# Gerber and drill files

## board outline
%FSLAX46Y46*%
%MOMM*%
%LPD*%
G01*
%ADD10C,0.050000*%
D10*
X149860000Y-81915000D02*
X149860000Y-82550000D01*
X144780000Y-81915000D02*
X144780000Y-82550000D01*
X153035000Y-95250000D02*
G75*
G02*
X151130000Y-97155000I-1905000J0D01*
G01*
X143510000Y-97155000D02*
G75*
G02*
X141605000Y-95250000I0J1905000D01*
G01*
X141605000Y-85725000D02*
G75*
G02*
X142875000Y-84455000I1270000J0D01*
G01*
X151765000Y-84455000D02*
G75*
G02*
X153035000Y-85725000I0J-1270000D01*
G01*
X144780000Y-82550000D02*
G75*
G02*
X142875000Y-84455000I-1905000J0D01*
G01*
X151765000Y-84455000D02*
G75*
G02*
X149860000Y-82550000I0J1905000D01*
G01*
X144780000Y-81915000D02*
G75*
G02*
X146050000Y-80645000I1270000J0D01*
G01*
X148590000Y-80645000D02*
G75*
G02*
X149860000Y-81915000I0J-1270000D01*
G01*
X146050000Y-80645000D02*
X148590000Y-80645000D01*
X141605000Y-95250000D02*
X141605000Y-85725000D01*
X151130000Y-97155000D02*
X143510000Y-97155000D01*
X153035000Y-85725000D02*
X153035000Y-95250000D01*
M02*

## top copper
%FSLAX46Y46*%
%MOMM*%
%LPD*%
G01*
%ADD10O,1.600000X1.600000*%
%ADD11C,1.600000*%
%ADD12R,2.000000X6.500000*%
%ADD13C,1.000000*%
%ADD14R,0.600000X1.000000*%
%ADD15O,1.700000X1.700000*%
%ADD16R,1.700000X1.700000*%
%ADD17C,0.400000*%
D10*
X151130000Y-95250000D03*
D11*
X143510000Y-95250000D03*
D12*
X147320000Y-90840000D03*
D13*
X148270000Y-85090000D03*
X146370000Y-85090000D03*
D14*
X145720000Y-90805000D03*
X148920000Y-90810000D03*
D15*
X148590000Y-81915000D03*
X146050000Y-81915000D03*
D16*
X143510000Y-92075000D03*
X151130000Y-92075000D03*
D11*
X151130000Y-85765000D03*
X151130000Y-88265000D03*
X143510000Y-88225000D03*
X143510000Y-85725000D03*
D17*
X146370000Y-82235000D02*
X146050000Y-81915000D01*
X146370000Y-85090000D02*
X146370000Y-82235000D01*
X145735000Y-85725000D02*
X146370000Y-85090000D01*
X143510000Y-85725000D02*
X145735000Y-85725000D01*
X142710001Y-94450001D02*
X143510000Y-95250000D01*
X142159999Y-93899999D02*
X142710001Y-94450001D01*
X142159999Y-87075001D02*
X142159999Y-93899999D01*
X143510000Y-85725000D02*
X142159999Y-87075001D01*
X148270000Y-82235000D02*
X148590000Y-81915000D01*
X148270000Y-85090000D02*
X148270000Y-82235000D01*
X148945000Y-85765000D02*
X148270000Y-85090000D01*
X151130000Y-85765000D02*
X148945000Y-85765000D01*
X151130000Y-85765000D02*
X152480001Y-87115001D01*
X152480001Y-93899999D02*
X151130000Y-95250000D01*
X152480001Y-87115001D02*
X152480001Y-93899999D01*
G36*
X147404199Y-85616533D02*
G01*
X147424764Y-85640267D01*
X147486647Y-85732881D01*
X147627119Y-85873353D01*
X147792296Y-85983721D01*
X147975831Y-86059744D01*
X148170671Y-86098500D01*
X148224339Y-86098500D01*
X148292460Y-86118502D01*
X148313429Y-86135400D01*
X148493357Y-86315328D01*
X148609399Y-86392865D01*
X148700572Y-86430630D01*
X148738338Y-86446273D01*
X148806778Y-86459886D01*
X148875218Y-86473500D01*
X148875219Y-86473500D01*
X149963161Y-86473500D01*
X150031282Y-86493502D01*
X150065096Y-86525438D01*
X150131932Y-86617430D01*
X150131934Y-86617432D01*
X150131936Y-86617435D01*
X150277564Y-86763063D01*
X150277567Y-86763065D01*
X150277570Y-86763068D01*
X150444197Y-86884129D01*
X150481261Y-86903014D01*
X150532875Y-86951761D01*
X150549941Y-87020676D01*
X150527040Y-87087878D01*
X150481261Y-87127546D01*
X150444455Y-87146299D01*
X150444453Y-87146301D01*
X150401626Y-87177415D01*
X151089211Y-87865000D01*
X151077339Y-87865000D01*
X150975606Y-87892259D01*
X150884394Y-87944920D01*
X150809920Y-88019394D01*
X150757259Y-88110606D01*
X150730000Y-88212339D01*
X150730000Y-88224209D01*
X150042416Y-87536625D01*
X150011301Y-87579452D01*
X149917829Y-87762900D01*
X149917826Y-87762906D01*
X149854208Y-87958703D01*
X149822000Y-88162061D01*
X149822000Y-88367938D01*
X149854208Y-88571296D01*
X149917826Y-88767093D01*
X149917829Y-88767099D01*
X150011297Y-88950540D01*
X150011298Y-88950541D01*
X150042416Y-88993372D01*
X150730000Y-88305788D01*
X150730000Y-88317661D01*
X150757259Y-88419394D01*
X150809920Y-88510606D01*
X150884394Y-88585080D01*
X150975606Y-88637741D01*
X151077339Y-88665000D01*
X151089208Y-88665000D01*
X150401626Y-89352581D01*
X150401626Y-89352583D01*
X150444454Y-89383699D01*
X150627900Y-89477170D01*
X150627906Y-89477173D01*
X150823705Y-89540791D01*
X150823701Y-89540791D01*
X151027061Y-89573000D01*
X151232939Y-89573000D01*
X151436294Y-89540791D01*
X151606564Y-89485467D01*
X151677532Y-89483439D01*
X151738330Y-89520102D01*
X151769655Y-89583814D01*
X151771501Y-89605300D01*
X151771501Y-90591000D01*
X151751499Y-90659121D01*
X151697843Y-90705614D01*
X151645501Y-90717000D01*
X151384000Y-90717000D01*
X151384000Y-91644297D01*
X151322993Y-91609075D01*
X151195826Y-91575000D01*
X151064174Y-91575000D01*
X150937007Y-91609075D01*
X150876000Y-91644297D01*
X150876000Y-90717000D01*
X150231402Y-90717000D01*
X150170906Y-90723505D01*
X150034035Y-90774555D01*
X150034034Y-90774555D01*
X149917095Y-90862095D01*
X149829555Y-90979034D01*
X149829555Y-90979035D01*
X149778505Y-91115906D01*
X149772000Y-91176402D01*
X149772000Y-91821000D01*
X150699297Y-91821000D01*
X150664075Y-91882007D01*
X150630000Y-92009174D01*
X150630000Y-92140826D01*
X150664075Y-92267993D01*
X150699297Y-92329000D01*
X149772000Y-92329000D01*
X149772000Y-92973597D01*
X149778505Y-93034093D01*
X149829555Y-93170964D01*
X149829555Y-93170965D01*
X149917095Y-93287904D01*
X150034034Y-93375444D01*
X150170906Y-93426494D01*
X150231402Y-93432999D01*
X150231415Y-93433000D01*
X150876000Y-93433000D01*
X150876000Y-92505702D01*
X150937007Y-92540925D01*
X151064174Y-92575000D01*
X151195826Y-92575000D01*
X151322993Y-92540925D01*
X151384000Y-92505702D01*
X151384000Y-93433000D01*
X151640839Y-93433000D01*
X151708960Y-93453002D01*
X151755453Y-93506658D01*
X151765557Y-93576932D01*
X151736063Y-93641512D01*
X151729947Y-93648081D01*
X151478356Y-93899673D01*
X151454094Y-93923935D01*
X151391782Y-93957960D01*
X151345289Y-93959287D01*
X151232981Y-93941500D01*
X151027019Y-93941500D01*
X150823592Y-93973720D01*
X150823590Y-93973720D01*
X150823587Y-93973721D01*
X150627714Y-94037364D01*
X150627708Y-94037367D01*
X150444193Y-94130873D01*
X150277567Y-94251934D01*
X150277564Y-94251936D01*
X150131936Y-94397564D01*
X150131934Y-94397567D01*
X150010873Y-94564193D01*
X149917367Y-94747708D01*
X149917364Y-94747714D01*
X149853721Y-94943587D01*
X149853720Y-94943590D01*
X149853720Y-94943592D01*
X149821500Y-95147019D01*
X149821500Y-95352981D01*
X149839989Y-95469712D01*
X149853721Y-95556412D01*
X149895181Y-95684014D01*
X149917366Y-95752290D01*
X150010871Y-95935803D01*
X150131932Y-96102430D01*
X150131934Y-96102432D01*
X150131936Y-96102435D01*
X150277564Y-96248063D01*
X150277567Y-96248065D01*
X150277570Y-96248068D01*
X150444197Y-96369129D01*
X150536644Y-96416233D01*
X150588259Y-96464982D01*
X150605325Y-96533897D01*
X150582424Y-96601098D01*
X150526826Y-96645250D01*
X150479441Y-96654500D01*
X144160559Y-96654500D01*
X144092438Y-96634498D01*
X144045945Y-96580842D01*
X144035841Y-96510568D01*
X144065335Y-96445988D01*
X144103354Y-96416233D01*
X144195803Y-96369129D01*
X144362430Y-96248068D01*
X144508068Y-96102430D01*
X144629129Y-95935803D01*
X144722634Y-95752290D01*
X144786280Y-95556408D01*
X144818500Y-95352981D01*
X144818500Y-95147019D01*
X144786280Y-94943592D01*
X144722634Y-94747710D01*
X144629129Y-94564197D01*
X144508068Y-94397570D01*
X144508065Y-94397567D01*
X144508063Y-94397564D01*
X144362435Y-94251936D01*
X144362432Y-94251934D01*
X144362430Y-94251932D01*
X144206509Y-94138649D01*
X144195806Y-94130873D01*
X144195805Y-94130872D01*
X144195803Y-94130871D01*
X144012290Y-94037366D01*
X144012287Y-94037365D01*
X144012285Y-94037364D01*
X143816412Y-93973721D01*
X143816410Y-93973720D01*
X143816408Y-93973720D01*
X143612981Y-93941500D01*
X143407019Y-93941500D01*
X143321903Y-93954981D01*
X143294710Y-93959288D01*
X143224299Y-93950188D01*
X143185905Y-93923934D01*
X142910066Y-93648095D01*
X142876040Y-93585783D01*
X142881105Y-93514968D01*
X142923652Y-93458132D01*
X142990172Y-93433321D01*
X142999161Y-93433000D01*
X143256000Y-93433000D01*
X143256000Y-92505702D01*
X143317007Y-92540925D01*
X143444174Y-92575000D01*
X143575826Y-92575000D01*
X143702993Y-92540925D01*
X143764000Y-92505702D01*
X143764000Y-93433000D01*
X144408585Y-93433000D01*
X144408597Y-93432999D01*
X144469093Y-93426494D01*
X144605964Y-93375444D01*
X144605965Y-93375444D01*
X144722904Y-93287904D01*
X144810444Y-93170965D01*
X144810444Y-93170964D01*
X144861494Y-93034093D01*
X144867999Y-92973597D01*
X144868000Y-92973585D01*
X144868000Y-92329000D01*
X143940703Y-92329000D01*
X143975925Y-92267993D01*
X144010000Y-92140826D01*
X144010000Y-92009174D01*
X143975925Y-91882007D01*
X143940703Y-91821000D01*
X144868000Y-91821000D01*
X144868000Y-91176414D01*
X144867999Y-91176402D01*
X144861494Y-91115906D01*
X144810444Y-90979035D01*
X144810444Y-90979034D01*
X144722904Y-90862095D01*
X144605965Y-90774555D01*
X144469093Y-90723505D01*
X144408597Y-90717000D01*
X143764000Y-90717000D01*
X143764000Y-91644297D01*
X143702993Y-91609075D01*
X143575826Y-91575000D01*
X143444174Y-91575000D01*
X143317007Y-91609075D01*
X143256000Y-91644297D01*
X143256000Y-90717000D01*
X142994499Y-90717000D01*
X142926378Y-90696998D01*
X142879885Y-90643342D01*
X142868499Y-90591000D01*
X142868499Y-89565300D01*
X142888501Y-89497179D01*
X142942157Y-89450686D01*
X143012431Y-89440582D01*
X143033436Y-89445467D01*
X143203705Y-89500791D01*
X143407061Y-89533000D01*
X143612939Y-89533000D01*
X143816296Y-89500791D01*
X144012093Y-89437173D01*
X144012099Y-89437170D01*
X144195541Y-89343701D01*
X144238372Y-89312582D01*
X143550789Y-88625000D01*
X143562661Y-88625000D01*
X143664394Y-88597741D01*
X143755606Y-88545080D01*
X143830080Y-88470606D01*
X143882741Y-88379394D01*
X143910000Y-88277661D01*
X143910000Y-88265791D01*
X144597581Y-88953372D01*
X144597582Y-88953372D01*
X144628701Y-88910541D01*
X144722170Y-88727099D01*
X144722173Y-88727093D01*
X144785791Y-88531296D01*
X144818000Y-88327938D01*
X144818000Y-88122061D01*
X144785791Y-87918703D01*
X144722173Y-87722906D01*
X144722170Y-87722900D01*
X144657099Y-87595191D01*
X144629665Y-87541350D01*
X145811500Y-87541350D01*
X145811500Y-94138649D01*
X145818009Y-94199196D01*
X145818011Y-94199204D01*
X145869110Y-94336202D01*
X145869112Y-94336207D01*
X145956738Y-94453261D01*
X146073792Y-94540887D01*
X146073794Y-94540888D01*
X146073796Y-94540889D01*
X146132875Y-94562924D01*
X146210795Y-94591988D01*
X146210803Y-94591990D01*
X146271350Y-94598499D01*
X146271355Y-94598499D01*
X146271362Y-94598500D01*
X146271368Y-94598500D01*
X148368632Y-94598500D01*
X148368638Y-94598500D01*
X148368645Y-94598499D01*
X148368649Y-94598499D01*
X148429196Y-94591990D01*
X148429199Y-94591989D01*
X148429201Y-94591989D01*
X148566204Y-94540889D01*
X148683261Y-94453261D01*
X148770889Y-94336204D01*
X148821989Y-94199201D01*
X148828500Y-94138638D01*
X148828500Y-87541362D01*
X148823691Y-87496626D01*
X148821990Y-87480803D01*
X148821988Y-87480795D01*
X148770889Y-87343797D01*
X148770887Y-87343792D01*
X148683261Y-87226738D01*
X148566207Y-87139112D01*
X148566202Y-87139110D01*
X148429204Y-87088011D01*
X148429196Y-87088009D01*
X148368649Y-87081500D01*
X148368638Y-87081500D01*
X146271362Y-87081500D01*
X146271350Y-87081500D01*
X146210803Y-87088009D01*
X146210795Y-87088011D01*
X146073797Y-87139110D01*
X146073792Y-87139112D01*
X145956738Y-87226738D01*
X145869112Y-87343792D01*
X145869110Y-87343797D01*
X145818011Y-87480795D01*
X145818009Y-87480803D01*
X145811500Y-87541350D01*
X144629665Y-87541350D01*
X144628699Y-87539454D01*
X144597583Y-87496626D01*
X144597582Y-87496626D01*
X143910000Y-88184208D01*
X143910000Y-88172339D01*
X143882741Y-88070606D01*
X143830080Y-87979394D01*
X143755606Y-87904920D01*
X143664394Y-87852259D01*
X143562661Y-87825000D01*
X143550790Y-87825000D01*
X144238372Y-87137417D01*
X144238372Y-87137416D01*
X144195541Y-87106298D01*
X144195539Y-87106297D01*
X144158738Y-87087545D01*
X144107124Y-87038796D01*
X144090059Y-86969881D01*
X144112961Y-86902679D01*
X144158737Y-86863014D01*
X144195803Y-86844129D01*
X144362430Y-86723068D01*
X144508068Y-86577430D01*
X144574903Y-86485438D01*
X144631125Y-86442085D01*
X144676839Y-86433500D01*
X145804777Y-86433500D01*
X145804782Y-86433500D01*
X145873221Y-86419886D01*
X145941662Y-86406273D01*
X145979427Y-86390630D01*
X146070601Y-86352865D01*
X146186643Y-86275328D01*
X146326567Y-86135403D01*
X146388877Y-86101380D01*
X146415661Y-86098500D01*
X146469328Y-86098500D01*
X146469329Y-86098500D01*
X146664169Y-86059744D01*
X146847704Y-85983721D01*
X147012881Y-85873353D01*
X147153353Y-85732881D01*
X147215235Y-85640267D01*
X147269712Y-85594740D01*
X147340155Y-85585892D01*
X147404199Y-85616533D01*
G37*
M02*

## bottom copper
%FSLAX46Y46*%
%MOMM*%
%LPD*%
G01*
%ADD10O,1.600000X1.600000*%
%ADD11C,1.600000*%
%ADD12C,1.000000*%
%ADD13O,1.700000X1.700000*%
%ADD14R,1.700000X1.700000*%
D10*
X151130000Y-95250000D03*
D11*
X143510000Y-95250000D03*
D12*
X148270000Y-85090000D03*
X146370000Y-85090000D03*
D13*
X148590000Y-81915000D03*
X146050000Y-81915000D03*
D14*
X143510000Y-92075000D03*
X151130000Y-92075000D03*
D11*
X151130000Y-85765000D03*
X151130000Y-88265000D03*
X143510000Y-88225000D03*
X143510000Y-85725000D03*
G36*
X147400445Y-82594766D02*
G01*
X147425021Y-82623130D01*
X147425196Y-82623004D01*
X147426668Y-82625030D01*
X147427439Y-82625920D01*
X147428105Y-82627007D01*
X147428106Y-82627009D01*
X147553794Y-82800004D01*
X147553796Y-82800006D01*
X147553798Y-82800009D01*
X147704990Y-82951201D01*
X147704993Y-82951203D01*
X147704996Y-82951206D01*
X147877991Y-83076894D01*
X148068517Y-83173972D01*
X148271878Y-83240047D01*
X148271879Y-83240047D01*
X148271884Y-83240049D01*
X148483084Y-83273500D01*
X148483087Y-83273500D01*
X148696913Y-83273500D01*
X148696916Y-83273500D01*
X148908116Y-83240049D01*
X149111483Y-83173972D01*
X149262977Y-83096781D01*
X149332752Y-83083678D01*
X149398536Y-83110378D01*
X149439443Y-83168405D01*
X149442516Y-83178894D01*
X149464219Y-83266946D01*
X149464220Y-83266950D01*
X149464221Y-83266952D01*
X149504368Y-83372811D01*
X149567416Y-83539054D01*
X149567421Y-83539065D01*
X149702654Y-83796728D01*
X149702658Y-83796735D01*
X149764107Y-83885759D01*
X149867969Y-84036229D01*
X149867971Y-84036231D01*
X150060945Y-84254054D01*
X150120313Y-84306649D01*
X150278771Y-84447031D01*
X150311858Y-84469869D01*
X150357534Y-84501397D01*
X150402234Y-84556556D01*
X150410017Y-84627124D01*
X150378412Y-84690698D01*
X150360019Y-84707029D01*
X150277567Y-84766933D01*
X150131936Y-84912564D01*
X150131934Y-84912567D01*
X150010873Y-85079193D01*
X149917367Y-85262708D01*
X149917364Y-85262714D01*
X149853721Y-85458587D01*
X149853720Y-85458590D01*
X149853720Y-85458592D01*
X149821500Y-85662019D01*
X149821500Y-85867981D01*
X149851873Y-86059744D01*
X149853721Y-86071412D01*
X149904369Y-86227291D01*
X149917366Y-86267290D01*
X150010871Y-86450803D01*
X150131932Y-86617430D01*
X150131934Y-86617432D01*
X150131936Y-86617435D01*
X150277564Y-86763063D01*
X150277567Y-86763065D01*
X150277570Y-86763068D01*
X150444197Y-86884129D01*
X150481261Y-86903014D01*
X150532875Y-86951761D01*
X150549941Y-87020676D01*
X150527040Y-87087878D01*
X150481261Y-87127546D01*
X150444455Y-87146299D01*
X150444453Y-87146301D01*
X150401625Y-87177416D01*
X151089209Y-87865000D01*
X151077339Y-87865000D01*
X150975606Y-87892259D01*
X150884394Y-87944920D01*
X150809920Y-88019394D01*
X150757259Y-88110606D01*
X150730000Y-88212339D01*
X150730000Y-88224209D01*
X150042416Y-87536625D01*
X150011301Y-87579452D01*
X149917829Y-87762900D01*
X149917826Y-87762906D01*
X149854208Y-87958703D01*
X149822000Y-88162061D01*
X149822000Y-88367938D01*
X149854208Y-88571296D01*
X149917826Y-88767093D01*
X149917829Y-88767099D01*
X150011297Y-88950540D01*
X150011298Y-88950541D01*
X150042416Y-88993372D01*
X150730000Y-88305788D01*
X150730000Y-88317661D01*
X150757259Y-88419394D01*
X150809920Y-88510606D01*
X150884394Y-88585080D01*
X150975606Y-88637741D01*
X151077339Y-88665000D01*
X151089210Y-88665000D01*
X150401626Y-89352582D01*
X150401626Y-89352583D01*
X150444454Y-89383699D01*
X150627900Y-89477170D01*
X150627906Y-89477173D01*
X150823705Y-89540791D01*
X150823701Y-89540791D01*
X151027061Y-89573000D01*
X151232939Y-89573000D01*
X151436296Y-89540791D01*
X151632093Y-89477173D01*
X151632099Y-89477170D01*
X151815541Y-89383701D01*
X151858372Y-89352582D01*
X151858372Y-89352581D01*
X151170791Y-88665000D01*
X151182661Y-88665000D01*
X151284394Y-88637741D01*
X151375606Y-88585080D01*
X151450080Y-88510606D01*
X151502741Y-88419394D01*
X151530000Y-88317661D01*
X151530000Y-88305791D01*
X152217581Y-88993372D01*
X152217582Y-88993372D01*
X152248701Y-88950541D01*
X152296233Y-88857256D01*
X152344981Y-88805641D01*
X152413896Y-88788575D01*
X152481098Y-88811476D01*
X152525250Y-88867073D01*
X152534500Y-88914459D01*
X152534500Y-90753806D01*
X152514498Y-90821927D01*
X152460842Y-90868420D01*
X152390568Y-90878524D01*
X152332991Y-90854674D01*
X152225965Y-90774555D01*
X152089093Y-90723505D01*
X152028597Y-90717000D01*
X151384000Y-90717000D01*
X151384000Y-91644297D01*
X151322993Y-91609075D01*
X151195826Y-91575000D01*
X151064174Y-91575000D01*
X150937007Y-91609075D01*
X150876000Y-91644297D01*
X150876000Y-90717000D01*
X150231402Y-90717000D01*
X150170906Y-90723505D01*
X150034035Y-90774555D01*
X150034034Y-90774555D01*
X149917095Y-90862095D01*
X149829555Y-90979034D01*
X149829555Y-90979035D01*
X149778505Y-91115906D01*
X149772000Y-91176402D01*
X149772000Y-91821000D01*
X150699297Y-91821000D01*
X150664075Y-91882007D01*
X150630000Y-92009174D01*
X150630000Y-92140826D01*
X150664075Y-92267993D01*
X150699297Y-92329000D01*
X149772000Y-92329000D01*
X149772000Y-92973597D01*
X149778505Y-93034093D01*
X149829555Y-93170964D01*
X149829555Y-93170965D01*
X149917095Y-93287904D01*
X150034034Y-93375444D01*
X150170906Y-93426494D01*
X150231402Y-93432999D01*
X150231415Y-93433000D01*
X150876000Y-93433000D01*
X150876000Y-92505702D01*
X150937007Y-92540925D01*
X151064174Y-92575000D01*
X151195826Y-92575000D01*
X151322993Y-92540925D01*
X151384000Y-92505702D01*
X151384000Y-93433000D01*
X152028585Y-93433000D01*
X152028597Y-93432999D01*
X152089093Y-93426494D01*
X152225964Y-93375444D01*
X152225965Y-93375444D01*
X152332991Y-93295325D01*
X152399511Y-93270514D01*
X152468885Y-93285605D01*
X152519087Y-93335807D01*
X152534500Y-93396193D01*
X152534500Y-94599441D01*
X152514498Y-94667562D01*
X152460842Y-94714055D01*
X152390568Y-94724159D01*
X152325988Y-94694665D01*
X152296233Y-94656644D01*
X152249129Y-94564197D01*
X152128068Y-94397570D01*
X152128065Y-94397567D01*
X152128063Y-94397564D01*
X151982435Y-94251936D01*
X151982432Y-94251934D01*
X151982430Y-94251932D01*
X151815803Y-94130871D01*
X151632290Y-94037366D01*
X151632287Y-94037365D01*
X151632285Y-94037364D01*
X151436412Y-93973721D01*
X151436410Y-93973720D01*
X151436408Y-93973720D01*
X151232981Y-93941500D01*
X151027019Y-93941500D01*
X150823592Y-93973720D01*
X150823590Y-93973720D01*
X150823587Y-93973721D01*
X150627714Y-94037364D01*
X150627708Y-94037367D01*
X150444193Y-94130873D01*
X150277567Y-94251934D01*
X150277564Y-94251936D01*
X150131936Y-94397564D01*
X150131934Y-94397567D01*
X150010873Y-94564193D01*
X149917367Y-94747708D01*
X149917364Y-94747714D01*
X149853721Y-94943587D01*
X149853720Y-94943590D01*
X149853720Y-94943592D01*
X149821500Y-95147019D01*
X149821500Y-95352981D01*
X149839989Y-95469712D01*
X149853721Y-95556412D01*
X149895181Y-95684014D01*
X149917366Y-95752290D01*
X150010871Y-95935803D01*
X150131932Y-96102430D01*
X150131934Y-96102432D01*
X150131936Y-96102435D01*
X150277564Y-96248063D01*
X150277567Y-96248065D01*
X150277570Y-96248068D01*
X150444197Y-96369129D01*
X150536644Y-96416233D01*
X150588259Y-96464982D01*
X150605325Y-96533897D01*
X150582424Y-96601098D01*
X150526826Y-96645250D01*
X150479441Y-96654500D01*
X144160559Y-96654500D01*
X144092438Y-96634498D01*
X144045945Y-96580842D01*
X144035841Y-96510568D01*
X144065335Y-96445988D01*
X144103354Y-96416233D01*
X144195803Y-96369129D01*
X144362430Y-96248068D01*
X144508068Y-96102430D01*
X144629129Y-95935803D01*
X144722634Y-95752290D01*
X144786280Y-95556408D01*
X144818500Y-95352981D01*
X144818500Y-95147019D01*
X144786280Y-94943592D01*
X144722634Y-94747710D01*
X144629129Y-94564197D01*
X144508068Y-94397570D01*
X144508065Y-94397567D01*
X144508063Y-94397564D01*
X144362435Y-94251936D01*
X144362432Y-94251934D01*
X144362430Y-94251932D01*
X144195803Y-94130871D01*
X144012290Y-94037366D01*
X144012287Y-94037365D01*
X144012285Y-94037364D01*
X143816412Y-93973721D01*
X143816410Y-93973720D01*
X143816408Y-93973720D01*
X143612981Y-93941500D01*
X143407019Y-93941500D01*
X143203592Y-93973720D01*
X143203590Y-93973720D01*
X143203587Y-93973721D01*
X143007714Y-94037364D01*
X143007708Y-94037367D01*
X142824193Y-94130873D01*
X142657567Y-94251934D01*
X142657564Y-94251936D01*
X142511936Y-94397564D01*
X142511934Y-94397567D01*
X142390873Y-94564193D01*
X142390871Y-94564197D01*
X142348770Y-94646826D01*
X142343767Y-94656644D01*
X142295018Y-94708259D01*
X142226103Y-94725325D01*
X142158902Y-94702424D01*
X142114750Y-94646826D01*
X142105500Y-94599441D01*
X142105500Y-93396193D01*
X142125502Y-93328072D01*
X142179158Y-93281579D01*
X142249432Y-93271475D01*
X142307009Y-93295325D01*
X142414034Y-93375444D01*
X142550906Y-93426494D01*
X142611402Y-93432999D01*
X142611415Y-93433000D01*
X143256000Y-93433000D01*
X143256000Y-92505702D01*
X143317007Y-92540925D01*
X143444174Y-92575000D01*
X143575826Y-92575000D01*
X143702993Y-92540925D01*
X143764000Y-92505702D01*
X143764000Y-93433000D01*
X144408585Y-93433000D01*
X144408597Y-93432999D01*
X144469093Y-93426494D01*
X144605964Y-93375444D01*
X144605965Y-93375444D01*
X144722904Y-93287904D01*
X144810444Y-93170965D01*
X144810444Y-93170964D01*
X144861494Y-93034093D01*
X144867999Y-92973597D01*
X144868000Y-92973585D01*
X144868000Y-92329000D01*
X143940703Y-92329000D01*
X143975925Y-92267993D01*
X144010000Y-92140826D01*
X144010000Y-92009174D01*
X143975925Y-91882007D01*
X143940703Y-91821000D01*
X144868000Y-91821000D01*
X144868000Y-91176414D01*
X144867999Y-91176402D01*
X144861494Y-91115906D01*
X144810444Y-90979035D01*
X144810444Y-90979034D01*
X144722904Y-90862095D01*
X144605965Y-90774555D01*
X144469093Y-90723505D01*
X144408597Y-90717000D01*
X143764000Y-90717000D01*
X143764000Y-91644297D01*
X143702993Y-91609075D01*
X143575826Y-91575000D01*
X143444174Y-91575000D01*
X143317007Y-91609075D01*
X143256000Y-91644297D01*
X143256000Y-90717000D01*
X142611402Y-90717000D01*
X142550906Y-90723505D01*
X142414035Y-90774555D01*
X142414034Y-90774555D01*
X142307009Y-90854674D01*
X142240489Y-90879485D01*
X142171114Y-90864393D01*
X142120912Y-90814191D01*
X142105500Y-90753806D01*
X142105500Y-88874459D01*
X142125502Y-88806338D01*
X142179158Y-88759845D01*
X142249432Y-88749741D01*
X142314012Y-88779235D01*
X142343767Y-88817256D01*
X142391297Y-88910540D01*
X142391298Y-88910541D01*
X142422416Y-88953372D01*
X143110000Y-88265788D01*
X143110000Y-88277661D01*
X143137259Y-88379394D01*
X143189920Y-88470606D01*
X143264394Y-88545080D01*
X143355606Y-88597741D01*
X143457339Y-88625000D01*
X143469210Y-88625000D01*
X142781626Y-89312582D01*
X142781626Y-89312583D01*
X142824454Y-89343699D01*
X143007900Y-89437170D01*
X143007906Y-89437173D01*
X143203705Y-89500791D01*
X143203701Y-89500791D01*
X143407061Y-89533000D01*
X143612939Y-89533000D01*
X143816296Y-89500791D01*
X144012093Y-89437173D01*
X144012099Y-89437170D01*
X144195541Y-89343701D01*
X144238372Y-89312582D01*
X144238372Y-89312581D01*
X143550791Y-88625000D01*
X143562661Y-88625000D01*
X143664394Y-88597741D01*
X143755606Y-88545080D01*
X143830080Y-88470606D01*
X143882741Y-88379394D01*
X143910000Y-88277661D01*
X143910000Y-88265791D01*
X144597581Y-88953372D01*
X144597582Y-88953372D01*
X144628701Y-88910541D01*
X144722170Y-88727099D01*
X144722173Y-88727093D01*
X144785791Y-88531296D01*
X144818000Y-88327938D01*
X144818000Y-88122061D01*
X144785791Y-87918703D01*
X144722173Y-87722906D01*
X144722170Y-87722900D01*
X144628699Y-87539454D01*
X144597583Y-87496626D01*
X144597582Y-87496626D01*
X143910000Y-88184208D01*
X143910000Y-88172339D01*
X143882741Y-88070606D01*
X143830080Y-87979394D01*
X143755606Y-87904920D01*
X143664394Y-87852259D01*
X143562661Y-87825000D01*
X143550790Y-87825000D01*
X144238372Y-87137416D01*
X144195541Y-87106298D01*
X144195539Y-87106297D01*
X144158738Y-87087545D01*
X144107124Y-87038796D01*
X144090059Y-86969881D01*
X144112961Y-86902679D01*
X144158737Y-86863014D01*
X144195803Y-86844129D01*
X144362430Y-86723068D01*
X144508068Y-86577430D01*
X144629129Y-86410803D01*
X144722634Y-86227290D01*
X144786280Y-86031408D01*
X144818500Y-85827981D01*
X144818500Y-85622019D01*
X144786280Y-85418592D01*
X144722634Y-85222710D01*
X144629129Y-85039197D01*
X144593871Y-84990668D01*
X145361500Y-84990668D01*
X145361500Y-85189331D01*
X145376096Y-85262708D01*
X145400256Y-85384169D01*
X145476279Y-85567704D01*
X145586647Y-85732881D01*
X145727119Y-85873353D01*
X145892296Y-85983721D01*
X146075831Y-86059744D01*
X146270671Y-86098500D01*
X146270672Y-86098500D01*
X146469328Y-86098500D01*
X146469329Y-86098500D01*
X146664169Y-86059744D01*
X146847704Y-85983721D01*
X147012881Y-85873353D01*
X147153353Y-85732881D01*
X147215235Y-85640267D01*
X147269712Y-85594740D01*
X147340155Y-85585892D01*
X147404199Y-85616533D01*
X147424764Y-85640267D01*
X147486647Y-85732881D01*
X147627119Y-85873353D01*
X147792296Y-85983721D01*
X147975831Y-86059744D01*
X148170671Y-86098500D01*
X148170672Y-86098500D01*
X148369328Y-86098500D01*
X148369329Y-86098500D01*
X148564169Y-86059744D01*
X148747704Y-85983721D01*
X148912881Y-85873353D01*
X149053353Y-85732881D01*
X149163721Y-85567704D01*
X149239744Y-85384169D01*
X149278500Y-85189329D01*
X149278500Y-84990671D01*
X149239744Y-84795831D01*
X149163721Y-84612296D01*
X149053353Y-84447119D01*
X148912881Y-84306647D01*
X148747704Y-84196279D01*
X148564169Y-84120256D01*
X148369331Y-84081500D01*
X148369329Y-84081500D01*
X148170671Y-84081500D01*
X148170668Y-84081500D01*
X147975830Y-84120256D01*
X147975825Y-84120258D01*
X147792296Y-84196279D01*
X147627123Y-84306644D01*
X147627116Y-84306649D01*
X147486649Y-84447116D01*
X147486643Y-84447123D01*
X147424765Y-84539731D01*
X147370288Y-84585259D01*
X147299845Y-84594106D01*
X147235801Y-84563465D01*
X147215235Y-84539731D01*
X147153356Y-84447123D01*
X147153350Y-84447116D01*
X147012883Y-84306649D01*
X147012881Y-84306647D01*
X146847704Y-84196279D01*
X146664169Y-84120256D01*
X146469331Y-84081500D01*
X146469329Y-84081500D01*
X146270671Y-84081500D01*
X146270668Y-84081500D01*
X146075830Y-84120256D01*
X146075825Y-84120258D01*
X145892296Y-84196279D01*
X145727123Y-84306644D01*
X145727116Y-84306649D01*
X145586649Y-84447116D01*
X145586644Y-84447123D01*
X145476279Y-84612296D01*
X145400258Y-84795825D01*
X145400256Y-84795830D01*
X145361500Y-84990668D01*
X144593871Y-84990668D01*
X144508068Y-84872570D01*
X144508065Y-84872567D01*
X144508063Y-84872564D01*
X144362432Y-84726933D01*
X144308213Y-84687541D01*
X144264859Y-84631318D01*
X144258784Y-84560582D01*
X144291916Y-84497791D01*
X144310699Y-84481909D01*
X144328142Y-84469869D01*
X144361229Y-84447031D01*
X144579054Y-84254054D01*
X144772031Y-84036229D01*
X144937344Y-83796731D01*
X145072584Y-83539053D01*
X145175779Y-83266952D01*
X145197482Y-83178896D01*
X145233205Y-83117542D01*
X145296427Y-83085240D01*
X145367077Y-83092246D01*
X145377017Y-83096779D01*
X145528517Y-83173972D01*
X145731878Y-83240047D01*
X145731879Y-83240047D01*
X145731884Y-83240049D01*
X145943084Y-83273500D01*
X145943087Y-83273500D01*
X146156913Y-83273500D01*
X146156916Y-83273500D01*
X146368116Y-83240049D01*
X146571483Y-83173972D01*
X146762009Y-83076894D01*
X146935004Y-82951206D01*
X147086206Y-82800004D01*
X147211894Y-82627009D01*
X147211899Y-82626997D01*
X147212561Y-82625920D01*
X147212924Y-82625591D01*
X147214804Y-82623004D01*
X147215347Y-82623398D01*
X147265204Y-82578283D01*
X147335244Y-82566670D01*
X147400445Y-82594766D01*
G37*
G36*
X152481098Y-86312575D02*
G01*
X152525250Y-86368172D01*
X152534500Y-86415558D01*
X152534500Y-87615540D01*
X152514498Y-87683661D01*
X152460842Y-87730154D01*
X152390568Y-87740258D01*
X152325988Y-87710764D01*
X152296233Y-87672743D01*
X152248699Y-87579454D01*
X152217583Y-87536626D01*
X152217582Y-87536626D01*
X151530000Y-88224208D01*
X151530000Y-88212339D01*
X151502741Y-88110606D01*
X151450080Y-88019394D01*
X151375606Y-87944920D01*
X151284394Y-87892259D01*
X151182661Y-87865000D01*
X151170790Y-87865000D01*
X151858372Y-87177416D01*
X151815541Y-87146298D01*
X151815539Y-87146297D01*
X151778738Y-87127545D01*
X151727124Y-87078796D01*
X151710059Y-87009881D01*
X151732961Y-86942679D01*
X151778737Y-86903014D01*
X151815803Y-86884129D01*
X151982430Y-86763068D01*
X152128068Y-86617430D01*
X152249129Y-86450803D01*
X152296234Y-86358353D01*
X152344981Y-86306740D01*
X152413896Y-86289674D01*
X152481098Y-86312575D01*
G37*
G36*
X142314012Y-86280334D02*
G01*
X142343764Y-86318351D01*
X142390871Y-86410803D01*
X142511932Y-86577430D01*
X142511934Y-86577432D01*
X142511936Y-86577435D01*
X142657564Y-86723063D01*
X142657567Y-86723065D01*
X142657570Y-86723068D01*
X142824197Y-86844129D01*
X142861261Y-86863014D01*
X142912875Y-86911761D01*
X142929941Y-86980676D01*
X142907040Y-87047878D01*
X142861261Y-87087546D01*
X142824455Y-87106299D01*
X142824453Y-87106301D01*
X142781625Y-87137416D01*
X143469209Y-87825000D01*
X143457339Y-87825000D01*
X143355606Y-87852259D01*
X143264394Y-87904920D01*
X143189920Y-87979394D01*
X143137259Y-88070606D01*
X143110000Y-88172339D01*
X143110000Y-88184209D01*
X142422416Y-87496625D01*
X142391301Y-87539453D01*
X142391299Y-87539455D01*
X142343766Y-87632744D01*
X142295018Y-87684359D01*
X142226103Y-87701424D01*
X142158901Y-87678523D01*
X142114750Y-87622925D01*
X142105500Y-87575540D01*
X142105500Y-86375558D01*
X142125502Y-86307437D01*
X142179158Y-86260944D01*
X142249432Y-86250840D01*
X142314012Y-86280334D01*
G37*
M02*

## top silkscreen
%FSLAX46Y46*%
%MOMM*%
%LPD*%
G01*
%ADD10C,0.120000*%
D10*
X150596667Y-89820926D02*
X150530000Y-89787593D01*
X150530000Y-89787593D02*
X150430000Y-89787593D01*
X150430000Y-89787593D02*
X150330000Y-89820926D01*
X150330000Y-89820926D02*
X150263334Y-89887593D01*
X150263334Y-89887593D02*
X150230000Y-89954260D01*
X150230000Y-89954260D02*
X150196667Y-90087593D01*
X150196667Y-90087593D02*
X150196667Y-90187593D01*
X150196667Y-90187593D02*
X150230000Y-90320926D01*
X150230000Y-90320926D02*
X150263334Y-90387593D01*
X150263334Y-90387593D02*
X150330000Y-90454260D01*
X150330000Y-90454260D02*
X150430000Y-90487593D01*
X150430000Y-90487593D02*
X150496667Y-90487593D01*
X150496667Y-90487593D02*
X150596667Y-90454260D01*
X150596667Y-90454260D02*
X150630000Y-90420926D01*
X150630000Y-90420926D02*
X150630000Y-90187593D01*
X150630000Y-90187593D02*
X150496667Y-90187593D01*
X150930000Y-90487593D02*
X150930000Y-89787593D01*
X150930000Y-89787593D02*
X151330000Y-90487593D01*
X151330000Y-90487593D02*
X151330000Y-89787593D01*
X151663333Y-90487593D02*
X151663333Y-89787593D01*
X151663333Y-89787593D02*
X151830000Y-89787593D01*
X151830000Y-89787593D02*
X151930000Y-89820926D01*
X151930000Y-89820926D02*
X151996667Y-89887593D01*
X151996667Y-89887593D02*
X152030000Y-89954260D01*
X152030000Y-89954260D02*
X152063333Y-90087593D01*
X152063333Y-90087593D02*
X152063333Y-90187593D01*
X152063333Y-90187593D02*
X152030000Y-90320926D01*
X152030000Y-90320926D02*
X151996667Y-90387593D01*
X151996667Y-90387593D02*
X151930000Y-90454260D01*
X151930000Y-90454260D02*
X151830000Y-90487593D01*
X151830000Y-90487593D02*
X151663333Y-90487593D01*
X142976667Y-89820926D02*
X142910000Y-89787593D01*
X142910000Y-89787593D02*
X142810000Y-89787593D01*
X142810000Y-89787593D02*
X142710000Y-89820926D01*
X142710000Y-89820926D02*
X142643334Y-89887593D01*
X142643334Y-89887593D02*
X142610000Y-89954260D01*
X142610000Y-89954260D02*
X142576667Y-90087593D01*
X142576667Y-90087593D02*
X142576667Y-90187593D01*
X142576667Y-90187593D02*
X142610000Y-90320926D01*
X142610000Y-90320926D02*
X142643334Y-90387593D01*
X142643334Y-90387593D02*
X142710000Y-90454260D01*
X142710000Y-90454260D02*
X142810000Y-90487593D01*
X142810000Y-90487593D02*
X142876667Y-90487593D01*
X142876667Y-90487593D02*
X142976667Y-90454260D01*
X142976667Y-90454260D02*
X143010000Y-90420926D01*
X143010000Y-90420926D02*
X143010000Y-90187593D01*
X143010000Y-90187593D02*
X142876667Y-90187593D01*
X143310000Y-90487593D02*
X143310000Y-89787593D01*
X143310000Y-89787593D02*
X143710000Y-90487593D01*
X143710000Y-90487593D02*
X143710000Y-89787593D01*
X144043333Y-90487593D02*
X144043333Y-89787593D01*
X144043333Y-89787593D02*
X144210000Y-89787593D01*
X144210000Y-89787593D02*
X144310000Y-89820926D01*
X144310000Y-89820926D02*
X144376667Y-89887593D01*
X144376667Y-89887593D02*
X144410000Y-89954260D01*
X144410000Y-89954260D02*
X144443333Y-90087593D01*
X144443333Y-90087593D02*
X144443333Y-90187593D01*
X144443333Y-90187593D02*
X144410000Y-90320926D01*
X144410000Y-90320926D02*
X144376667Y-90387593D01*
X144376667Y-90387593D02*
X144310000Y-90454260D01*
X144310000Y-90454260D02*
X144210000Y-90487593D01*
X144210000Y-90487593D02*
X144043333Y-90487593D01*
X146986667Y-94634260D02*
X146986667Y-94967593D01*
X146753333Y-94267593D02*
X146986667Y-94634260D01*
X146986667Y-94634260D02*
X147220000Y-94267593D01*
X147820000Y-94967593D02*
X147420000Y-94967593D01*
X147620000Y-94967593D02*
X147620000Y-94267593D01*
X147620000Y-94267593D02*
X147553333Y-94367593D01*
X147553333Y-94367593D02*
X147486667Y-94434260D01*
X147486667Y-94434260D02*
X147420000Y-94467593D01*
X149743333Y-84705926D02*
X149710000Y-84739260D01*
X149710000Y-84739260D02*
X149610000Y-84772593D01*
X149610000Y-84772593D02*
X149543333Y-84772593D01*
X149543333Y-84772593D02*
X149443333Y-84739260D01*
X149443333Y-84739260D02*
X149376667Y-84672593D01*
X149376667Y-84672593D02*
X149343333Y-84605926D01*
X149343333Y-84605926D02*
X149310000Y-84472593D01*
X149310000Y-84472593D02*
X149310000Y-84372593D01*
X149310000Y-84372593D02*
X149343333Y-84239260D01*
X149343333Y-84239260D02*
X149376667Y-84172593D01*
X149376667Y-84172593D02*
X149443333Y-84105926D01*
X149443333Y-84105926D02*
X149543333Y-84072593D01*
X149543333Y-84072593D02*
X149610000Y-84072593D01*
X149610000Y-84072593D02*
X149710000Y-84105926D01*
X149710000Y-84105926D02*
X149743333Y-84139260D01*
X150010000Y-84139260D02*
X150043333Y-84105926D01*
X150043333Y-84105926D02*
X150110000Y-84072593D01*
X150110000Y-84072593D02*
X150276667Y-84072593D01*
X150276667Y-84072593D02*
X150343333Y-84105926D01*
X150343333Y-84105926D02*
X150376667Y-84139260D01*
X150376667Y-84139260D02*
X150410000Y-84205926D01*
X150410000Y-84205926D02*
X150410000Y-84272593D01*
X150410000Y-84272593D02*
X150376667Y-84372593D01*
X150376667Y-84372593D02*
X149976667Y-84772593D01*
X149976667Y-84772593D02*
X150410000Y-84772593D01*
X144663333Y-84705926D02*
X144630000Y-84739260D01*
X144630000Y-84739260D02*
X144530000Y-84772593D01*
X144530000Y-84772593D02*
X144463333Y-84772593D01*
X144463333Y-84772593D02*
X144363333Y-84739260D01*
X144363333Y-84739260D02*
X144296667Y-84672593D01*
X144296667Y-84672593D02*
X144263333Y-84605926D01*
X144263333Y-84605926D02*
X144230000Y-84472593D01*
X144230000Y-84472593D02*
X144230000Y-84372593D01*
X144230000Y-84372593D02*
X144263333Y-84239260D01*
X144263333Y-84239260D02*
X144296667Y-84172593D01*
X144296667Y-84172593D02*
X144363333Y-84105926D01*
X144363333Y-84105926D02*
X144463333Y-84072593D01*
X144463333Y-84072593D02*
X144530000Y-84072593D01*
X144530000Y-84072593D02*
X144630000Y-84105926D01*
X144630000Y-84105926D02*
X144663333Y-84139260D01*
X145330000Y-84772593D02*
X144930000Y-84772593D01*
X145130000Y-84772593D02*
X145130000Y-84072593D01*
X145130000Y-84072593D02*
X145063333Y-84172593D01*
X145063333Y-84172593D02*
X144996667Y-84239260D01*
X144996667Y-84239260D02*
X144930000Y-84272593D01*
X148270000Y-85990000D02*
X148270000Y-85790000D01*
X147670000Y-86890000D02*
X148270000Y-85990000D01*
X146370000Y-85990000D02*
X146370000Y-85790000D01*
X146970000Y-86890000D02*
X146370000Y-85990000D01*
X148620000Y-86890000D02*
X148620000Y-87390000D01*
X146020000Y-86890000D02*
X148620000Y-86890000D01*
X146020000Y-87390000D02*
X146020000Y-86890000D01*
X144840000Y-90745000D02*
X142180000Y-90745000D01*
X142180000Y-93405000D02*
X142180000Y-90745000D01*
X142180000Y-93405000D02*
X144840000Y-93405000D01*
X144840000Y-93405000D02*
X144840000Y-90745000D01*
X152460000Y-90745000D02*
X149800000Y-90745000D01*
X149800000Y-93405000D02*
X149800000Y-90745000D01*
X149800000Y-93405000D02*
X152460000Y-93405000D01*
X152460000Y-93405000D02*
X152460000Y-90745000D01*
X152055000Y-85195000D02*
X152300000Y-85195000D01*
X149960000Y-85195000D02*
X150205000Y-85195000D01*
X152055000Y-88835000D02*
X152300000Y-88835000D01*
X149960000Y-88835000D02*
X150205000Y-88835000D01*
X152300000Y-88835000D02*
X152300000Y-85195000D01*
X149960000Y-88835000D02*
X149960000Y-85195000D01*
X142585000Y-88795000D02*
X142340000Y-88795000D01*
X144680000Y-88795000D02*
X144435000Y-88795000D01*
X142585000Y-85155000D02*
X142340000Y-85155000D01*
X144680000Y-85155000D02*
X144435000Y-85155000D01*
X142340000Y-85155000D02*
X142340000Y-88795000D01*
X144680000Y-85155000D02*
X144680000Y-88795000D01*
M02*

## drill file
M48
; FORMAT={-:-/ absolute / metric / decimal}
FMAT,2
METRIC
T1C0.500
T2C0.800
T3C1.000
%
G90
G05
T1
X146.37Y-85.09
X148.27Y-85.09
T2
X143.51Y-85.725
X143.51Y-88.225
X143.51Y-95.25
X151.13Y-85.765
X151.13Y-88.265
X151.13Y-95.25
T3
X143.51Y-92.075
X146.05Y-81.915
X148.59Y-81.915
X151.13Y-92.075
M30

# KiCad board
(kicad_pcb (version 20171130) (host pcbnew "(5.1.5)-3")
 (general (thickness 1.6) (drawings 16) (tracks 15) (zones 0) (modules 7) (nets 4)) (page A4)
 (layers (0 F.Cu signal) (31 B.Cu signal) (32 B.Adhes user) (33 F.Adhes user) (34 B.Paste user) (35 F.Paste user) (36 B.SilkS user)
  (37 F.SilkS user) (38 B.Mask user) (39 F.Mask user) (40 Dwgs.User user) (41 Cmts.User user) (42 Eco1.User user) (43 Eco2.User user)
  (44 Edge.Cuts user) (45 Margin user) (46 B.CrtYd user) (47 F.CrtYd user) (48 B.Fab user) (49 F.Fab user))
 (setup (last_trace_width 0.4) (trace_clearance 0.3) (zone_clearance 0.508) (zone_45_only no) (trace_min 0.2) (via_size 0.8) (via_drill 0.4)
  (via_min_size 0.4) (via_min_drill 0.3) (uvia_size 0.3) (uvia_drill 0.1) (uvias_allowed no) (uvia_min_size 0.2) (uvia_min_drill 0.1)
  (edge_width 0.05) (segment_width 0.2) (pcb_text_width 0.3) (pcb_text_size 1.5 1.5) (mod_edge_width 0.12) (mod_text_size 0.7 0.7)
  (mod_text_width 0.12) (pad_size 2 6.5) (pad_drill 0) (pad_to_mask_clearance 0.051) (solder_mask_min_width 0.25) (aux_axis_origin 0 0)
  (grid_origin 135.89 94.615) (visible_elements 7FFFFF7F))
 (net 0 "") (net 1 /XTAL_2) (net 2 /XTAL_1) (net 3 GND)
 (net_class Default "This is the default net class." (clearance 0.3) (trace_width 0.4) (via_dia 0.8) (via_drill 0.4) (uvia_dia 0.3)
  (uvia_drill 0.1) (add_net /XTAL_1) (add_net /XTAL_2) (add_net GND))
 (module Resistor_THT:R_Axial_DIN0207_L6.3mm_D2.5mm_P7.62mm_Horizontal (layer B.Cu) (at 143.51 95.25)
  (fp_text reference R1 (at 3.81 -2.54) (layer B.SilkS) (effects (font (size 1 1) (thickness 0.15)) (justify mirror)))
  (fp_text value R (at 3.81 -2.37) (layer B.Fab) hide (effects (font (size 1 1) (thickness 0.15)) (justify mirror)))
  (pad 2 thru_hole oval (at 7.62 0) (size 1.6 1.6) (drill 0.8) (layers *.Cu *.Mask) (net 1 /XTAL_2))
  (pad 1 thru_hole circle (at 0 0) (size 1.6 1.6) (drill 0.8) (layers *.Cu *.Mask) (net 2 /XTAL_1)))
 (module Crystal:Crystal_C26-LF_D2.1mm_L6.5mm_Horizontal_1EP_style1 (layer F.Cu) (at 146.37 85.09)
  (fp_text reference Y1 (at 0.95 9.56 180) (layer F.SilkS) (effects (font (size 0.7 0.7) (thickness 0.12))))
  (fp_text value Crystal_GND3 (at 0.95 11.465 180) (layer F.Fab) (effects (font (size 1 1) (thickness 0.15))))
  (fp_line (start 1.9 0.9) (end 1.9 0.7) (layer F.SilkS) (width 0.12))
  (fp_line (start 1.3 1.8) (end 1.9 0.9) (layer F.SilkS) (width 0.12))
  (fp_line (start 0 0.9) (end 0 0.7) (layer F.SilkS) (width 0.12))
  (fp_line (start 0.6 1.8) (end 0 0.9) (layer F.SilkS) (width 0.12))
  (fp_line (start 2.25 1.8) (end 2.25 2.3) (layer F.SilkS) (width 0.12))
  (fp_line (start -0.35 1.8) (end 2.25 1.8) (layer F.SilkS) (width 0.12))
  (fp_line (start -0.35 2.3) (end -0.35 1.8) (layer F.SilkS) (width 0.12))
  (pad NC smd rect (at 0.95 5.75) (size 2 6.5) (layers F.Cu F.Paste F.Mask))
  (pad 2 thru_hole circle (at 1.9 0) (size 1 1) (drill 0.5) (layers *.Cu *.Mask) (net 1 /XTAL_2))
  (pad 1 thru_hole circle (at 0 0) (size 1 1) (drill 0.5) (layers *.Cu *.Mask) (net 2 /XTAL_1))
  (pad 3 smd rect (at -0.65 5.715) (size 0.6 1) (layers F.Cu F.Paste F.Mask) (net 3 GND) (zone_connect 2))
  (pad 3 smd rect (at 2.55 5.72) (size 0.6 1) (layers F.Cu F.Paste F.Mask) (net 3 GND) (zone_connect 2)))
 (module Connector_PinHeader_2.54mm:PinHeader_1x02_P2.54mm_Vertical (layer B.Cu) (at 146.05 81.915 270)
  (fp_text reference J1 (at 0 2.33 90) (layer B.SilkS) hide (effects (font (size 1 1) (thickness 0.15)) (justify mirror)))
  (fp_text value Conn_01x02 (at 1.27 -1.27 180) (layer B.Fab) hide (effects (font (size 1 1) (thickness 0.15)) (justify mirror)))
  (pad 2 thru_hole oval (at 0 -2.54 270) (size 1.7 1.7) (drill 1) (layers *.Cu *.Mask) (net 1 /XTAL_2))
  (pad 1 thru_hole oval (at 0 0 270) (size 1.7 1.7) (drill 1) (layers *.Cu *.Mask) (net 2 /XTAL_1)))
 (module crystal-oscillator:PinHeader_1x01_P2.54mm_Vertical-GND (layer B.Cu) (at 143.51 92.075 90)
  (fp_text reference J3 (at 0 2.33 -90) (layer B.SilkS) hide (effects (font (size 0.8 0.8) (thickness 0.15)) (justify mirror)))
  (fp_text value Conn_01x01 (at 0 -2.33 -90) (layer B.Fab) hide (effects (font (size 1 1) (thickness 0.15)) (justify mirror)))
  (fp_line (start 1.33 1.33) (end 1.33 -1.33) (layer F.SilkS) (width 0.12))
  (fp_line (start -1.33 -1.33) (end 1.33 -1.33) (layer F.SilkS) (width 0.12))
  (fp_line (start -1.33 -1.33) (end -1.33 1.33) (layer F.SilkS) (width 0.12))
  (fp_line (start -1.33 1.33) (end 1.33 1.33) (layer F.SilkS) (width 0.12))
  (pad 1 thru_hole rect (at 0 0 90) (size 1.7 1.7) (drill 1) (layers *.Cu *.Mask) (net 3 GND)))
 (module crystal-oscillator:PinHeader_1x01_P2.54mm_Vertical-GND (layer B.Cu) (at 151.13 92.075 90)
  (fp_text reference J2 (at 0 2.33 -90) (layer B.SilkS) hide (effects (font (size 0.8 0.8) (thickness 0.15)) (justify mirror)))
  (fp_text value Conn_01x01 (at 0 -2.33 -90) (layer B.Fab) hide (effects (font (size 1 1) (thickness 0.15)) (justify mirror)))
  (fp_line (start 1.33 1.33) (end 1.33 -1.33) (layer F.SilkS) (width 0.12))
  (fp_line (start -1.33 -1.33) (end 1.33 -1.33) (layer F.SilkS) (width 0.12))
  (fp_line (start -1.33 -1.33) (end -1.33 1.33) (layer F.SilkS) (width 0.12))
  (fp_line (start -1.33 1.33) (end 1.33 1.33) (layer F.SilkS) (width 0.12))
  (pad 1 thru_hole rect (at 0 0 90) (size 1.7 1.7) (drill 1) (layers *.Cu *.Mask) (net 3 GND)))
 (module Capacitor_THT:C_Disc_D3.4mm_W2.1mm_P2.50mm (layer F.Cu) (at 151.13 88.265 90)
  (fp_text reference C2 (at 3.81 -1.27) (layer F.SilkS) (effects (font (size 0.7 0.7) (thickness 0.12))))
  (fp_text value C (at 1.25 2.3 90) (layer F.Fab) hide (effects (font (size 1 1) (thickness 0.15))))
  (fp_line (start 3.07 0.925) (end 3.07 1.17) (layer F.SilkS) (width 0.12))
  (fp_line (start 3.07 -1.17) (end 3.07 -0.925) (layer F.SilkS) (width 0.12))
  (fp_line (start -0.57 0.925) (end -0.57 1.17) (layer F.SilkS) (width 0.12))
  (fp_line (start -0.57 -1.17) (end -0.57 -0.925) (layer F.SilkS) (width 0.12))
  (fp_line (start -0.57 1.17) (end 3.07 1.17) (layer F.SilkS) (width 0.12))
  (fp_line (start -0.57 -1.17) (end 3.07 -1.17) (layer F.SilkS) (width 0.12))
  (pad 2 thru_hole circle (at 2.5 0 90) (size 1.6 1.6) (drill 0.8) (layers *.Cu *.Mask) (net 1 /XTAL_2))
  (pad 1 thru_hole circle (at 0 0 90) (size 1.6 1.6) (drill 0.8) (layers *.Cu *.Mask) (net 3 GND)))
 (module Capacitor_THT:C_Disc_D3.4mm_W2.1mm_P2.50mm (layer F.Cu) (at 143.51 85.725 270)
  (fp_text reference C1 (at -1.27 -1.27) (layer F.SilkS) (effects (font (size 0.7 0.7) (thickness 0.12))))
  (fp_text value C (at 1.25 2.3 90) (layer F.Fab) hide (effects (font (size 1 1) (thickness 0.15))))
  (fp_line (start 3.07 0.925) (end 3.07 1.17) (layer F.SilkS) (width 0.12))
  (fp_line (start 3.07 -1.17) (end 3.07 -0.925) (layer F.SilkS) (width 0.12))
  (fp_line (start -0.57 0.925) (end -0.57 1.17) (layer F.SilkS) (width 0.12))
  (fp_line (start -0.57 -1.17) (end -0.57 -0.925) (layer F.SilkS) (width 0.12))
  (fp_line (start -0.57 1.17) (end 3.07 1.17) (layer F.SilkS) (width 0.12))
  (fp_line (start -0.57 -1.17) (end 3.07 -1.17) (layer F.SilkS) (width 0.12))
  (pad 2 thru_hole circle (at 2.5 0 270) (size 1.6 1.6) (drill 0.8) (layers *.Cu *.Mask) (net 3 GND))
  (pad 1 thru_hole circle (at 0 0 270) (size 1.6 1.6) (drill 0.8) (layers *.Cu *.Mask) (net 2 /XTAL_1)))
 (gr_line (start 149.86 81.915) (end 149.86 82.55) (layer Edge.Cuts) (width 0.05))
 (gr_line (start 144.78 81.915) (end 144.78 82.55) (layer Edge.Cuts) (width 0.05))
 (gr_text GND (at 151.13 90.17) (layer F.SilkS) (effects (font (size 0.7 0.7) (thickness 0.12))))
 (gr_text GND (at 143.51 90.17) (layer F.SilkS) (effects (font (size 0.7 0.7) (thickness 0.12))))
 (gr_arc (start 151.13 95.25) (end 151.13 97.155) (angle -90) (layer Edge.Cuts) (width 0.05))
 (gr_arc (start 143.51 95.25) (end 141.605 95.25) (angle -90) (layer Edge.Cuts) (width 0.05))
 (gr_arc (start 142.875 85.725) (end 142.875 84.455) (angle -90) (layer Edge.Cuts) (width 0.05))
 (gr_arc (start 151.765 85.725) (end 153.035 85.725) (angle -90) (layer Edge.Cuts) (width 0.05))
 (gr_arc (start 142.875 82.55) (end 142.875 84.455) (angle -90) (layer Edge.Cuts) (width 0.05))
 (gr_arc (start 151.765 82.55) (end 149.86 82.55) (angle -90) (layer Edge.Cuts) (width 0.05))
 (gr_arc (start 146.05 81.915) (end 146.05 80.645) (angle -90) (layer Edge.Cuts) (width 0.05))
 (gr_arc (start 148.59 81.915) (end 149.86 81.915) (angle -90) (layer Edge.Cuts) (width 0.05))
 (gr_line (start 146.05 80.645) (end 148.59 80.645) (layer Edge.Cuts) (width 0.05))
 (gr_line (start 141.605 95.25) (end 141.605 85.725) (layer Edge.Cuts) (width 0.05))
 (gr_line (start 151.13 97.155) (end 143.51 97.155) (layer Edge.Cuts) (width 0.05))
 (gr_line (start 153.035 85.725) (end 153.035 95.25) (layer Edge.Cuts) (width 0.05))
 (segment (start 146.37 82.235) (end 146.05 81.915) (width 0.4) (layer F.Cu) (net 2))
 (segment (start 146.37 85.09) (end 146.37 82.235) (width 0.4) (layer F.Cu) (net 2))
 (segment (start 145.735 85.725) (end 146.37 85.09) (width 0.4) (layer F.Cu) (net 2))
 (segment (start 143.51 85.725) (end 145.735 85.725) (width 0.4) (layer F.Cu) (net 2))
 (segment (start 142.710001 94.450001) (end 143.51 95.25) (width 0.4) (layer F.Cu) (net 2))
 (segment (start 142.159999 93.899999) (end 142.710001 94.450001) (width 0.4) (layer F.Cu) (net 2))
 (segment (start 142.159999 87.075001) (end 142.159999 93.899999) (width 0.4) (layer F.Cu) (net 2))
 (segment (start 143.51 85.725) (end 142.159999 87.075001) (width 0.4) (layer F.Cu) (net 2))
 (segment (start 148.27 82.235) (end 148.59 81.915) (width 0.4) (layer F.Cu) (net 1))
 (segment (start 148.27 85.09) (end 148.27 82.235) (width 0.4) (layer F.Cu) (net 1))
 (segment (start 148.945 85.765) (end 148.27 85.09) (width 0.4) (layer F.Cu) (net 1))
 (segment (start 151.13 85.765) (end 148.945 85.765) (width 0.4) (layer F.Cu) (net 1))
 (segment (start 151.13 85.765) (end 152.480001 87.115001) (width 0.4) (layer F.Cu) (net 1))
 (segment (start 152.480001 93.899999) (end 151.13 95.25) (width 0.4) (layer F.Cu) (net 1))
 (segment (start 152.480001 87.115001) (end 152.480001 93.899999) (width 0.4) (layer F.Cu) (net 1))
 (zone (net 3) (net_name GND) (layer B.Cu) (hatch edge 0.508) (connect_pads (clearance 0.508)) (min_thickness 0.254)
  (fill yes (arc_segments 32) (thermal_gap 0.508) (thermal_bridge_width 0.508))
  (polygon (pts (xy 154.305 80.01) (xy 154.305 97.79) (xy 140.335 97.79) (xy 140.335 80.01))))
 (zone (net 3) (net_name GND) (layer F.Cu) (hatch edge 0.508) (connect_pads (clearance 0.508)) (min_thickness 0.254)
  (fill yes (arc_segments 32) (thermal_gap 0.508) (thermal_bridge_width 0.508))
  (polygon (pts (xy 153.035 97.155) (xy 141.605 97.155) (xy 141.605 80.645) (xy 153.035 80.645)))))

